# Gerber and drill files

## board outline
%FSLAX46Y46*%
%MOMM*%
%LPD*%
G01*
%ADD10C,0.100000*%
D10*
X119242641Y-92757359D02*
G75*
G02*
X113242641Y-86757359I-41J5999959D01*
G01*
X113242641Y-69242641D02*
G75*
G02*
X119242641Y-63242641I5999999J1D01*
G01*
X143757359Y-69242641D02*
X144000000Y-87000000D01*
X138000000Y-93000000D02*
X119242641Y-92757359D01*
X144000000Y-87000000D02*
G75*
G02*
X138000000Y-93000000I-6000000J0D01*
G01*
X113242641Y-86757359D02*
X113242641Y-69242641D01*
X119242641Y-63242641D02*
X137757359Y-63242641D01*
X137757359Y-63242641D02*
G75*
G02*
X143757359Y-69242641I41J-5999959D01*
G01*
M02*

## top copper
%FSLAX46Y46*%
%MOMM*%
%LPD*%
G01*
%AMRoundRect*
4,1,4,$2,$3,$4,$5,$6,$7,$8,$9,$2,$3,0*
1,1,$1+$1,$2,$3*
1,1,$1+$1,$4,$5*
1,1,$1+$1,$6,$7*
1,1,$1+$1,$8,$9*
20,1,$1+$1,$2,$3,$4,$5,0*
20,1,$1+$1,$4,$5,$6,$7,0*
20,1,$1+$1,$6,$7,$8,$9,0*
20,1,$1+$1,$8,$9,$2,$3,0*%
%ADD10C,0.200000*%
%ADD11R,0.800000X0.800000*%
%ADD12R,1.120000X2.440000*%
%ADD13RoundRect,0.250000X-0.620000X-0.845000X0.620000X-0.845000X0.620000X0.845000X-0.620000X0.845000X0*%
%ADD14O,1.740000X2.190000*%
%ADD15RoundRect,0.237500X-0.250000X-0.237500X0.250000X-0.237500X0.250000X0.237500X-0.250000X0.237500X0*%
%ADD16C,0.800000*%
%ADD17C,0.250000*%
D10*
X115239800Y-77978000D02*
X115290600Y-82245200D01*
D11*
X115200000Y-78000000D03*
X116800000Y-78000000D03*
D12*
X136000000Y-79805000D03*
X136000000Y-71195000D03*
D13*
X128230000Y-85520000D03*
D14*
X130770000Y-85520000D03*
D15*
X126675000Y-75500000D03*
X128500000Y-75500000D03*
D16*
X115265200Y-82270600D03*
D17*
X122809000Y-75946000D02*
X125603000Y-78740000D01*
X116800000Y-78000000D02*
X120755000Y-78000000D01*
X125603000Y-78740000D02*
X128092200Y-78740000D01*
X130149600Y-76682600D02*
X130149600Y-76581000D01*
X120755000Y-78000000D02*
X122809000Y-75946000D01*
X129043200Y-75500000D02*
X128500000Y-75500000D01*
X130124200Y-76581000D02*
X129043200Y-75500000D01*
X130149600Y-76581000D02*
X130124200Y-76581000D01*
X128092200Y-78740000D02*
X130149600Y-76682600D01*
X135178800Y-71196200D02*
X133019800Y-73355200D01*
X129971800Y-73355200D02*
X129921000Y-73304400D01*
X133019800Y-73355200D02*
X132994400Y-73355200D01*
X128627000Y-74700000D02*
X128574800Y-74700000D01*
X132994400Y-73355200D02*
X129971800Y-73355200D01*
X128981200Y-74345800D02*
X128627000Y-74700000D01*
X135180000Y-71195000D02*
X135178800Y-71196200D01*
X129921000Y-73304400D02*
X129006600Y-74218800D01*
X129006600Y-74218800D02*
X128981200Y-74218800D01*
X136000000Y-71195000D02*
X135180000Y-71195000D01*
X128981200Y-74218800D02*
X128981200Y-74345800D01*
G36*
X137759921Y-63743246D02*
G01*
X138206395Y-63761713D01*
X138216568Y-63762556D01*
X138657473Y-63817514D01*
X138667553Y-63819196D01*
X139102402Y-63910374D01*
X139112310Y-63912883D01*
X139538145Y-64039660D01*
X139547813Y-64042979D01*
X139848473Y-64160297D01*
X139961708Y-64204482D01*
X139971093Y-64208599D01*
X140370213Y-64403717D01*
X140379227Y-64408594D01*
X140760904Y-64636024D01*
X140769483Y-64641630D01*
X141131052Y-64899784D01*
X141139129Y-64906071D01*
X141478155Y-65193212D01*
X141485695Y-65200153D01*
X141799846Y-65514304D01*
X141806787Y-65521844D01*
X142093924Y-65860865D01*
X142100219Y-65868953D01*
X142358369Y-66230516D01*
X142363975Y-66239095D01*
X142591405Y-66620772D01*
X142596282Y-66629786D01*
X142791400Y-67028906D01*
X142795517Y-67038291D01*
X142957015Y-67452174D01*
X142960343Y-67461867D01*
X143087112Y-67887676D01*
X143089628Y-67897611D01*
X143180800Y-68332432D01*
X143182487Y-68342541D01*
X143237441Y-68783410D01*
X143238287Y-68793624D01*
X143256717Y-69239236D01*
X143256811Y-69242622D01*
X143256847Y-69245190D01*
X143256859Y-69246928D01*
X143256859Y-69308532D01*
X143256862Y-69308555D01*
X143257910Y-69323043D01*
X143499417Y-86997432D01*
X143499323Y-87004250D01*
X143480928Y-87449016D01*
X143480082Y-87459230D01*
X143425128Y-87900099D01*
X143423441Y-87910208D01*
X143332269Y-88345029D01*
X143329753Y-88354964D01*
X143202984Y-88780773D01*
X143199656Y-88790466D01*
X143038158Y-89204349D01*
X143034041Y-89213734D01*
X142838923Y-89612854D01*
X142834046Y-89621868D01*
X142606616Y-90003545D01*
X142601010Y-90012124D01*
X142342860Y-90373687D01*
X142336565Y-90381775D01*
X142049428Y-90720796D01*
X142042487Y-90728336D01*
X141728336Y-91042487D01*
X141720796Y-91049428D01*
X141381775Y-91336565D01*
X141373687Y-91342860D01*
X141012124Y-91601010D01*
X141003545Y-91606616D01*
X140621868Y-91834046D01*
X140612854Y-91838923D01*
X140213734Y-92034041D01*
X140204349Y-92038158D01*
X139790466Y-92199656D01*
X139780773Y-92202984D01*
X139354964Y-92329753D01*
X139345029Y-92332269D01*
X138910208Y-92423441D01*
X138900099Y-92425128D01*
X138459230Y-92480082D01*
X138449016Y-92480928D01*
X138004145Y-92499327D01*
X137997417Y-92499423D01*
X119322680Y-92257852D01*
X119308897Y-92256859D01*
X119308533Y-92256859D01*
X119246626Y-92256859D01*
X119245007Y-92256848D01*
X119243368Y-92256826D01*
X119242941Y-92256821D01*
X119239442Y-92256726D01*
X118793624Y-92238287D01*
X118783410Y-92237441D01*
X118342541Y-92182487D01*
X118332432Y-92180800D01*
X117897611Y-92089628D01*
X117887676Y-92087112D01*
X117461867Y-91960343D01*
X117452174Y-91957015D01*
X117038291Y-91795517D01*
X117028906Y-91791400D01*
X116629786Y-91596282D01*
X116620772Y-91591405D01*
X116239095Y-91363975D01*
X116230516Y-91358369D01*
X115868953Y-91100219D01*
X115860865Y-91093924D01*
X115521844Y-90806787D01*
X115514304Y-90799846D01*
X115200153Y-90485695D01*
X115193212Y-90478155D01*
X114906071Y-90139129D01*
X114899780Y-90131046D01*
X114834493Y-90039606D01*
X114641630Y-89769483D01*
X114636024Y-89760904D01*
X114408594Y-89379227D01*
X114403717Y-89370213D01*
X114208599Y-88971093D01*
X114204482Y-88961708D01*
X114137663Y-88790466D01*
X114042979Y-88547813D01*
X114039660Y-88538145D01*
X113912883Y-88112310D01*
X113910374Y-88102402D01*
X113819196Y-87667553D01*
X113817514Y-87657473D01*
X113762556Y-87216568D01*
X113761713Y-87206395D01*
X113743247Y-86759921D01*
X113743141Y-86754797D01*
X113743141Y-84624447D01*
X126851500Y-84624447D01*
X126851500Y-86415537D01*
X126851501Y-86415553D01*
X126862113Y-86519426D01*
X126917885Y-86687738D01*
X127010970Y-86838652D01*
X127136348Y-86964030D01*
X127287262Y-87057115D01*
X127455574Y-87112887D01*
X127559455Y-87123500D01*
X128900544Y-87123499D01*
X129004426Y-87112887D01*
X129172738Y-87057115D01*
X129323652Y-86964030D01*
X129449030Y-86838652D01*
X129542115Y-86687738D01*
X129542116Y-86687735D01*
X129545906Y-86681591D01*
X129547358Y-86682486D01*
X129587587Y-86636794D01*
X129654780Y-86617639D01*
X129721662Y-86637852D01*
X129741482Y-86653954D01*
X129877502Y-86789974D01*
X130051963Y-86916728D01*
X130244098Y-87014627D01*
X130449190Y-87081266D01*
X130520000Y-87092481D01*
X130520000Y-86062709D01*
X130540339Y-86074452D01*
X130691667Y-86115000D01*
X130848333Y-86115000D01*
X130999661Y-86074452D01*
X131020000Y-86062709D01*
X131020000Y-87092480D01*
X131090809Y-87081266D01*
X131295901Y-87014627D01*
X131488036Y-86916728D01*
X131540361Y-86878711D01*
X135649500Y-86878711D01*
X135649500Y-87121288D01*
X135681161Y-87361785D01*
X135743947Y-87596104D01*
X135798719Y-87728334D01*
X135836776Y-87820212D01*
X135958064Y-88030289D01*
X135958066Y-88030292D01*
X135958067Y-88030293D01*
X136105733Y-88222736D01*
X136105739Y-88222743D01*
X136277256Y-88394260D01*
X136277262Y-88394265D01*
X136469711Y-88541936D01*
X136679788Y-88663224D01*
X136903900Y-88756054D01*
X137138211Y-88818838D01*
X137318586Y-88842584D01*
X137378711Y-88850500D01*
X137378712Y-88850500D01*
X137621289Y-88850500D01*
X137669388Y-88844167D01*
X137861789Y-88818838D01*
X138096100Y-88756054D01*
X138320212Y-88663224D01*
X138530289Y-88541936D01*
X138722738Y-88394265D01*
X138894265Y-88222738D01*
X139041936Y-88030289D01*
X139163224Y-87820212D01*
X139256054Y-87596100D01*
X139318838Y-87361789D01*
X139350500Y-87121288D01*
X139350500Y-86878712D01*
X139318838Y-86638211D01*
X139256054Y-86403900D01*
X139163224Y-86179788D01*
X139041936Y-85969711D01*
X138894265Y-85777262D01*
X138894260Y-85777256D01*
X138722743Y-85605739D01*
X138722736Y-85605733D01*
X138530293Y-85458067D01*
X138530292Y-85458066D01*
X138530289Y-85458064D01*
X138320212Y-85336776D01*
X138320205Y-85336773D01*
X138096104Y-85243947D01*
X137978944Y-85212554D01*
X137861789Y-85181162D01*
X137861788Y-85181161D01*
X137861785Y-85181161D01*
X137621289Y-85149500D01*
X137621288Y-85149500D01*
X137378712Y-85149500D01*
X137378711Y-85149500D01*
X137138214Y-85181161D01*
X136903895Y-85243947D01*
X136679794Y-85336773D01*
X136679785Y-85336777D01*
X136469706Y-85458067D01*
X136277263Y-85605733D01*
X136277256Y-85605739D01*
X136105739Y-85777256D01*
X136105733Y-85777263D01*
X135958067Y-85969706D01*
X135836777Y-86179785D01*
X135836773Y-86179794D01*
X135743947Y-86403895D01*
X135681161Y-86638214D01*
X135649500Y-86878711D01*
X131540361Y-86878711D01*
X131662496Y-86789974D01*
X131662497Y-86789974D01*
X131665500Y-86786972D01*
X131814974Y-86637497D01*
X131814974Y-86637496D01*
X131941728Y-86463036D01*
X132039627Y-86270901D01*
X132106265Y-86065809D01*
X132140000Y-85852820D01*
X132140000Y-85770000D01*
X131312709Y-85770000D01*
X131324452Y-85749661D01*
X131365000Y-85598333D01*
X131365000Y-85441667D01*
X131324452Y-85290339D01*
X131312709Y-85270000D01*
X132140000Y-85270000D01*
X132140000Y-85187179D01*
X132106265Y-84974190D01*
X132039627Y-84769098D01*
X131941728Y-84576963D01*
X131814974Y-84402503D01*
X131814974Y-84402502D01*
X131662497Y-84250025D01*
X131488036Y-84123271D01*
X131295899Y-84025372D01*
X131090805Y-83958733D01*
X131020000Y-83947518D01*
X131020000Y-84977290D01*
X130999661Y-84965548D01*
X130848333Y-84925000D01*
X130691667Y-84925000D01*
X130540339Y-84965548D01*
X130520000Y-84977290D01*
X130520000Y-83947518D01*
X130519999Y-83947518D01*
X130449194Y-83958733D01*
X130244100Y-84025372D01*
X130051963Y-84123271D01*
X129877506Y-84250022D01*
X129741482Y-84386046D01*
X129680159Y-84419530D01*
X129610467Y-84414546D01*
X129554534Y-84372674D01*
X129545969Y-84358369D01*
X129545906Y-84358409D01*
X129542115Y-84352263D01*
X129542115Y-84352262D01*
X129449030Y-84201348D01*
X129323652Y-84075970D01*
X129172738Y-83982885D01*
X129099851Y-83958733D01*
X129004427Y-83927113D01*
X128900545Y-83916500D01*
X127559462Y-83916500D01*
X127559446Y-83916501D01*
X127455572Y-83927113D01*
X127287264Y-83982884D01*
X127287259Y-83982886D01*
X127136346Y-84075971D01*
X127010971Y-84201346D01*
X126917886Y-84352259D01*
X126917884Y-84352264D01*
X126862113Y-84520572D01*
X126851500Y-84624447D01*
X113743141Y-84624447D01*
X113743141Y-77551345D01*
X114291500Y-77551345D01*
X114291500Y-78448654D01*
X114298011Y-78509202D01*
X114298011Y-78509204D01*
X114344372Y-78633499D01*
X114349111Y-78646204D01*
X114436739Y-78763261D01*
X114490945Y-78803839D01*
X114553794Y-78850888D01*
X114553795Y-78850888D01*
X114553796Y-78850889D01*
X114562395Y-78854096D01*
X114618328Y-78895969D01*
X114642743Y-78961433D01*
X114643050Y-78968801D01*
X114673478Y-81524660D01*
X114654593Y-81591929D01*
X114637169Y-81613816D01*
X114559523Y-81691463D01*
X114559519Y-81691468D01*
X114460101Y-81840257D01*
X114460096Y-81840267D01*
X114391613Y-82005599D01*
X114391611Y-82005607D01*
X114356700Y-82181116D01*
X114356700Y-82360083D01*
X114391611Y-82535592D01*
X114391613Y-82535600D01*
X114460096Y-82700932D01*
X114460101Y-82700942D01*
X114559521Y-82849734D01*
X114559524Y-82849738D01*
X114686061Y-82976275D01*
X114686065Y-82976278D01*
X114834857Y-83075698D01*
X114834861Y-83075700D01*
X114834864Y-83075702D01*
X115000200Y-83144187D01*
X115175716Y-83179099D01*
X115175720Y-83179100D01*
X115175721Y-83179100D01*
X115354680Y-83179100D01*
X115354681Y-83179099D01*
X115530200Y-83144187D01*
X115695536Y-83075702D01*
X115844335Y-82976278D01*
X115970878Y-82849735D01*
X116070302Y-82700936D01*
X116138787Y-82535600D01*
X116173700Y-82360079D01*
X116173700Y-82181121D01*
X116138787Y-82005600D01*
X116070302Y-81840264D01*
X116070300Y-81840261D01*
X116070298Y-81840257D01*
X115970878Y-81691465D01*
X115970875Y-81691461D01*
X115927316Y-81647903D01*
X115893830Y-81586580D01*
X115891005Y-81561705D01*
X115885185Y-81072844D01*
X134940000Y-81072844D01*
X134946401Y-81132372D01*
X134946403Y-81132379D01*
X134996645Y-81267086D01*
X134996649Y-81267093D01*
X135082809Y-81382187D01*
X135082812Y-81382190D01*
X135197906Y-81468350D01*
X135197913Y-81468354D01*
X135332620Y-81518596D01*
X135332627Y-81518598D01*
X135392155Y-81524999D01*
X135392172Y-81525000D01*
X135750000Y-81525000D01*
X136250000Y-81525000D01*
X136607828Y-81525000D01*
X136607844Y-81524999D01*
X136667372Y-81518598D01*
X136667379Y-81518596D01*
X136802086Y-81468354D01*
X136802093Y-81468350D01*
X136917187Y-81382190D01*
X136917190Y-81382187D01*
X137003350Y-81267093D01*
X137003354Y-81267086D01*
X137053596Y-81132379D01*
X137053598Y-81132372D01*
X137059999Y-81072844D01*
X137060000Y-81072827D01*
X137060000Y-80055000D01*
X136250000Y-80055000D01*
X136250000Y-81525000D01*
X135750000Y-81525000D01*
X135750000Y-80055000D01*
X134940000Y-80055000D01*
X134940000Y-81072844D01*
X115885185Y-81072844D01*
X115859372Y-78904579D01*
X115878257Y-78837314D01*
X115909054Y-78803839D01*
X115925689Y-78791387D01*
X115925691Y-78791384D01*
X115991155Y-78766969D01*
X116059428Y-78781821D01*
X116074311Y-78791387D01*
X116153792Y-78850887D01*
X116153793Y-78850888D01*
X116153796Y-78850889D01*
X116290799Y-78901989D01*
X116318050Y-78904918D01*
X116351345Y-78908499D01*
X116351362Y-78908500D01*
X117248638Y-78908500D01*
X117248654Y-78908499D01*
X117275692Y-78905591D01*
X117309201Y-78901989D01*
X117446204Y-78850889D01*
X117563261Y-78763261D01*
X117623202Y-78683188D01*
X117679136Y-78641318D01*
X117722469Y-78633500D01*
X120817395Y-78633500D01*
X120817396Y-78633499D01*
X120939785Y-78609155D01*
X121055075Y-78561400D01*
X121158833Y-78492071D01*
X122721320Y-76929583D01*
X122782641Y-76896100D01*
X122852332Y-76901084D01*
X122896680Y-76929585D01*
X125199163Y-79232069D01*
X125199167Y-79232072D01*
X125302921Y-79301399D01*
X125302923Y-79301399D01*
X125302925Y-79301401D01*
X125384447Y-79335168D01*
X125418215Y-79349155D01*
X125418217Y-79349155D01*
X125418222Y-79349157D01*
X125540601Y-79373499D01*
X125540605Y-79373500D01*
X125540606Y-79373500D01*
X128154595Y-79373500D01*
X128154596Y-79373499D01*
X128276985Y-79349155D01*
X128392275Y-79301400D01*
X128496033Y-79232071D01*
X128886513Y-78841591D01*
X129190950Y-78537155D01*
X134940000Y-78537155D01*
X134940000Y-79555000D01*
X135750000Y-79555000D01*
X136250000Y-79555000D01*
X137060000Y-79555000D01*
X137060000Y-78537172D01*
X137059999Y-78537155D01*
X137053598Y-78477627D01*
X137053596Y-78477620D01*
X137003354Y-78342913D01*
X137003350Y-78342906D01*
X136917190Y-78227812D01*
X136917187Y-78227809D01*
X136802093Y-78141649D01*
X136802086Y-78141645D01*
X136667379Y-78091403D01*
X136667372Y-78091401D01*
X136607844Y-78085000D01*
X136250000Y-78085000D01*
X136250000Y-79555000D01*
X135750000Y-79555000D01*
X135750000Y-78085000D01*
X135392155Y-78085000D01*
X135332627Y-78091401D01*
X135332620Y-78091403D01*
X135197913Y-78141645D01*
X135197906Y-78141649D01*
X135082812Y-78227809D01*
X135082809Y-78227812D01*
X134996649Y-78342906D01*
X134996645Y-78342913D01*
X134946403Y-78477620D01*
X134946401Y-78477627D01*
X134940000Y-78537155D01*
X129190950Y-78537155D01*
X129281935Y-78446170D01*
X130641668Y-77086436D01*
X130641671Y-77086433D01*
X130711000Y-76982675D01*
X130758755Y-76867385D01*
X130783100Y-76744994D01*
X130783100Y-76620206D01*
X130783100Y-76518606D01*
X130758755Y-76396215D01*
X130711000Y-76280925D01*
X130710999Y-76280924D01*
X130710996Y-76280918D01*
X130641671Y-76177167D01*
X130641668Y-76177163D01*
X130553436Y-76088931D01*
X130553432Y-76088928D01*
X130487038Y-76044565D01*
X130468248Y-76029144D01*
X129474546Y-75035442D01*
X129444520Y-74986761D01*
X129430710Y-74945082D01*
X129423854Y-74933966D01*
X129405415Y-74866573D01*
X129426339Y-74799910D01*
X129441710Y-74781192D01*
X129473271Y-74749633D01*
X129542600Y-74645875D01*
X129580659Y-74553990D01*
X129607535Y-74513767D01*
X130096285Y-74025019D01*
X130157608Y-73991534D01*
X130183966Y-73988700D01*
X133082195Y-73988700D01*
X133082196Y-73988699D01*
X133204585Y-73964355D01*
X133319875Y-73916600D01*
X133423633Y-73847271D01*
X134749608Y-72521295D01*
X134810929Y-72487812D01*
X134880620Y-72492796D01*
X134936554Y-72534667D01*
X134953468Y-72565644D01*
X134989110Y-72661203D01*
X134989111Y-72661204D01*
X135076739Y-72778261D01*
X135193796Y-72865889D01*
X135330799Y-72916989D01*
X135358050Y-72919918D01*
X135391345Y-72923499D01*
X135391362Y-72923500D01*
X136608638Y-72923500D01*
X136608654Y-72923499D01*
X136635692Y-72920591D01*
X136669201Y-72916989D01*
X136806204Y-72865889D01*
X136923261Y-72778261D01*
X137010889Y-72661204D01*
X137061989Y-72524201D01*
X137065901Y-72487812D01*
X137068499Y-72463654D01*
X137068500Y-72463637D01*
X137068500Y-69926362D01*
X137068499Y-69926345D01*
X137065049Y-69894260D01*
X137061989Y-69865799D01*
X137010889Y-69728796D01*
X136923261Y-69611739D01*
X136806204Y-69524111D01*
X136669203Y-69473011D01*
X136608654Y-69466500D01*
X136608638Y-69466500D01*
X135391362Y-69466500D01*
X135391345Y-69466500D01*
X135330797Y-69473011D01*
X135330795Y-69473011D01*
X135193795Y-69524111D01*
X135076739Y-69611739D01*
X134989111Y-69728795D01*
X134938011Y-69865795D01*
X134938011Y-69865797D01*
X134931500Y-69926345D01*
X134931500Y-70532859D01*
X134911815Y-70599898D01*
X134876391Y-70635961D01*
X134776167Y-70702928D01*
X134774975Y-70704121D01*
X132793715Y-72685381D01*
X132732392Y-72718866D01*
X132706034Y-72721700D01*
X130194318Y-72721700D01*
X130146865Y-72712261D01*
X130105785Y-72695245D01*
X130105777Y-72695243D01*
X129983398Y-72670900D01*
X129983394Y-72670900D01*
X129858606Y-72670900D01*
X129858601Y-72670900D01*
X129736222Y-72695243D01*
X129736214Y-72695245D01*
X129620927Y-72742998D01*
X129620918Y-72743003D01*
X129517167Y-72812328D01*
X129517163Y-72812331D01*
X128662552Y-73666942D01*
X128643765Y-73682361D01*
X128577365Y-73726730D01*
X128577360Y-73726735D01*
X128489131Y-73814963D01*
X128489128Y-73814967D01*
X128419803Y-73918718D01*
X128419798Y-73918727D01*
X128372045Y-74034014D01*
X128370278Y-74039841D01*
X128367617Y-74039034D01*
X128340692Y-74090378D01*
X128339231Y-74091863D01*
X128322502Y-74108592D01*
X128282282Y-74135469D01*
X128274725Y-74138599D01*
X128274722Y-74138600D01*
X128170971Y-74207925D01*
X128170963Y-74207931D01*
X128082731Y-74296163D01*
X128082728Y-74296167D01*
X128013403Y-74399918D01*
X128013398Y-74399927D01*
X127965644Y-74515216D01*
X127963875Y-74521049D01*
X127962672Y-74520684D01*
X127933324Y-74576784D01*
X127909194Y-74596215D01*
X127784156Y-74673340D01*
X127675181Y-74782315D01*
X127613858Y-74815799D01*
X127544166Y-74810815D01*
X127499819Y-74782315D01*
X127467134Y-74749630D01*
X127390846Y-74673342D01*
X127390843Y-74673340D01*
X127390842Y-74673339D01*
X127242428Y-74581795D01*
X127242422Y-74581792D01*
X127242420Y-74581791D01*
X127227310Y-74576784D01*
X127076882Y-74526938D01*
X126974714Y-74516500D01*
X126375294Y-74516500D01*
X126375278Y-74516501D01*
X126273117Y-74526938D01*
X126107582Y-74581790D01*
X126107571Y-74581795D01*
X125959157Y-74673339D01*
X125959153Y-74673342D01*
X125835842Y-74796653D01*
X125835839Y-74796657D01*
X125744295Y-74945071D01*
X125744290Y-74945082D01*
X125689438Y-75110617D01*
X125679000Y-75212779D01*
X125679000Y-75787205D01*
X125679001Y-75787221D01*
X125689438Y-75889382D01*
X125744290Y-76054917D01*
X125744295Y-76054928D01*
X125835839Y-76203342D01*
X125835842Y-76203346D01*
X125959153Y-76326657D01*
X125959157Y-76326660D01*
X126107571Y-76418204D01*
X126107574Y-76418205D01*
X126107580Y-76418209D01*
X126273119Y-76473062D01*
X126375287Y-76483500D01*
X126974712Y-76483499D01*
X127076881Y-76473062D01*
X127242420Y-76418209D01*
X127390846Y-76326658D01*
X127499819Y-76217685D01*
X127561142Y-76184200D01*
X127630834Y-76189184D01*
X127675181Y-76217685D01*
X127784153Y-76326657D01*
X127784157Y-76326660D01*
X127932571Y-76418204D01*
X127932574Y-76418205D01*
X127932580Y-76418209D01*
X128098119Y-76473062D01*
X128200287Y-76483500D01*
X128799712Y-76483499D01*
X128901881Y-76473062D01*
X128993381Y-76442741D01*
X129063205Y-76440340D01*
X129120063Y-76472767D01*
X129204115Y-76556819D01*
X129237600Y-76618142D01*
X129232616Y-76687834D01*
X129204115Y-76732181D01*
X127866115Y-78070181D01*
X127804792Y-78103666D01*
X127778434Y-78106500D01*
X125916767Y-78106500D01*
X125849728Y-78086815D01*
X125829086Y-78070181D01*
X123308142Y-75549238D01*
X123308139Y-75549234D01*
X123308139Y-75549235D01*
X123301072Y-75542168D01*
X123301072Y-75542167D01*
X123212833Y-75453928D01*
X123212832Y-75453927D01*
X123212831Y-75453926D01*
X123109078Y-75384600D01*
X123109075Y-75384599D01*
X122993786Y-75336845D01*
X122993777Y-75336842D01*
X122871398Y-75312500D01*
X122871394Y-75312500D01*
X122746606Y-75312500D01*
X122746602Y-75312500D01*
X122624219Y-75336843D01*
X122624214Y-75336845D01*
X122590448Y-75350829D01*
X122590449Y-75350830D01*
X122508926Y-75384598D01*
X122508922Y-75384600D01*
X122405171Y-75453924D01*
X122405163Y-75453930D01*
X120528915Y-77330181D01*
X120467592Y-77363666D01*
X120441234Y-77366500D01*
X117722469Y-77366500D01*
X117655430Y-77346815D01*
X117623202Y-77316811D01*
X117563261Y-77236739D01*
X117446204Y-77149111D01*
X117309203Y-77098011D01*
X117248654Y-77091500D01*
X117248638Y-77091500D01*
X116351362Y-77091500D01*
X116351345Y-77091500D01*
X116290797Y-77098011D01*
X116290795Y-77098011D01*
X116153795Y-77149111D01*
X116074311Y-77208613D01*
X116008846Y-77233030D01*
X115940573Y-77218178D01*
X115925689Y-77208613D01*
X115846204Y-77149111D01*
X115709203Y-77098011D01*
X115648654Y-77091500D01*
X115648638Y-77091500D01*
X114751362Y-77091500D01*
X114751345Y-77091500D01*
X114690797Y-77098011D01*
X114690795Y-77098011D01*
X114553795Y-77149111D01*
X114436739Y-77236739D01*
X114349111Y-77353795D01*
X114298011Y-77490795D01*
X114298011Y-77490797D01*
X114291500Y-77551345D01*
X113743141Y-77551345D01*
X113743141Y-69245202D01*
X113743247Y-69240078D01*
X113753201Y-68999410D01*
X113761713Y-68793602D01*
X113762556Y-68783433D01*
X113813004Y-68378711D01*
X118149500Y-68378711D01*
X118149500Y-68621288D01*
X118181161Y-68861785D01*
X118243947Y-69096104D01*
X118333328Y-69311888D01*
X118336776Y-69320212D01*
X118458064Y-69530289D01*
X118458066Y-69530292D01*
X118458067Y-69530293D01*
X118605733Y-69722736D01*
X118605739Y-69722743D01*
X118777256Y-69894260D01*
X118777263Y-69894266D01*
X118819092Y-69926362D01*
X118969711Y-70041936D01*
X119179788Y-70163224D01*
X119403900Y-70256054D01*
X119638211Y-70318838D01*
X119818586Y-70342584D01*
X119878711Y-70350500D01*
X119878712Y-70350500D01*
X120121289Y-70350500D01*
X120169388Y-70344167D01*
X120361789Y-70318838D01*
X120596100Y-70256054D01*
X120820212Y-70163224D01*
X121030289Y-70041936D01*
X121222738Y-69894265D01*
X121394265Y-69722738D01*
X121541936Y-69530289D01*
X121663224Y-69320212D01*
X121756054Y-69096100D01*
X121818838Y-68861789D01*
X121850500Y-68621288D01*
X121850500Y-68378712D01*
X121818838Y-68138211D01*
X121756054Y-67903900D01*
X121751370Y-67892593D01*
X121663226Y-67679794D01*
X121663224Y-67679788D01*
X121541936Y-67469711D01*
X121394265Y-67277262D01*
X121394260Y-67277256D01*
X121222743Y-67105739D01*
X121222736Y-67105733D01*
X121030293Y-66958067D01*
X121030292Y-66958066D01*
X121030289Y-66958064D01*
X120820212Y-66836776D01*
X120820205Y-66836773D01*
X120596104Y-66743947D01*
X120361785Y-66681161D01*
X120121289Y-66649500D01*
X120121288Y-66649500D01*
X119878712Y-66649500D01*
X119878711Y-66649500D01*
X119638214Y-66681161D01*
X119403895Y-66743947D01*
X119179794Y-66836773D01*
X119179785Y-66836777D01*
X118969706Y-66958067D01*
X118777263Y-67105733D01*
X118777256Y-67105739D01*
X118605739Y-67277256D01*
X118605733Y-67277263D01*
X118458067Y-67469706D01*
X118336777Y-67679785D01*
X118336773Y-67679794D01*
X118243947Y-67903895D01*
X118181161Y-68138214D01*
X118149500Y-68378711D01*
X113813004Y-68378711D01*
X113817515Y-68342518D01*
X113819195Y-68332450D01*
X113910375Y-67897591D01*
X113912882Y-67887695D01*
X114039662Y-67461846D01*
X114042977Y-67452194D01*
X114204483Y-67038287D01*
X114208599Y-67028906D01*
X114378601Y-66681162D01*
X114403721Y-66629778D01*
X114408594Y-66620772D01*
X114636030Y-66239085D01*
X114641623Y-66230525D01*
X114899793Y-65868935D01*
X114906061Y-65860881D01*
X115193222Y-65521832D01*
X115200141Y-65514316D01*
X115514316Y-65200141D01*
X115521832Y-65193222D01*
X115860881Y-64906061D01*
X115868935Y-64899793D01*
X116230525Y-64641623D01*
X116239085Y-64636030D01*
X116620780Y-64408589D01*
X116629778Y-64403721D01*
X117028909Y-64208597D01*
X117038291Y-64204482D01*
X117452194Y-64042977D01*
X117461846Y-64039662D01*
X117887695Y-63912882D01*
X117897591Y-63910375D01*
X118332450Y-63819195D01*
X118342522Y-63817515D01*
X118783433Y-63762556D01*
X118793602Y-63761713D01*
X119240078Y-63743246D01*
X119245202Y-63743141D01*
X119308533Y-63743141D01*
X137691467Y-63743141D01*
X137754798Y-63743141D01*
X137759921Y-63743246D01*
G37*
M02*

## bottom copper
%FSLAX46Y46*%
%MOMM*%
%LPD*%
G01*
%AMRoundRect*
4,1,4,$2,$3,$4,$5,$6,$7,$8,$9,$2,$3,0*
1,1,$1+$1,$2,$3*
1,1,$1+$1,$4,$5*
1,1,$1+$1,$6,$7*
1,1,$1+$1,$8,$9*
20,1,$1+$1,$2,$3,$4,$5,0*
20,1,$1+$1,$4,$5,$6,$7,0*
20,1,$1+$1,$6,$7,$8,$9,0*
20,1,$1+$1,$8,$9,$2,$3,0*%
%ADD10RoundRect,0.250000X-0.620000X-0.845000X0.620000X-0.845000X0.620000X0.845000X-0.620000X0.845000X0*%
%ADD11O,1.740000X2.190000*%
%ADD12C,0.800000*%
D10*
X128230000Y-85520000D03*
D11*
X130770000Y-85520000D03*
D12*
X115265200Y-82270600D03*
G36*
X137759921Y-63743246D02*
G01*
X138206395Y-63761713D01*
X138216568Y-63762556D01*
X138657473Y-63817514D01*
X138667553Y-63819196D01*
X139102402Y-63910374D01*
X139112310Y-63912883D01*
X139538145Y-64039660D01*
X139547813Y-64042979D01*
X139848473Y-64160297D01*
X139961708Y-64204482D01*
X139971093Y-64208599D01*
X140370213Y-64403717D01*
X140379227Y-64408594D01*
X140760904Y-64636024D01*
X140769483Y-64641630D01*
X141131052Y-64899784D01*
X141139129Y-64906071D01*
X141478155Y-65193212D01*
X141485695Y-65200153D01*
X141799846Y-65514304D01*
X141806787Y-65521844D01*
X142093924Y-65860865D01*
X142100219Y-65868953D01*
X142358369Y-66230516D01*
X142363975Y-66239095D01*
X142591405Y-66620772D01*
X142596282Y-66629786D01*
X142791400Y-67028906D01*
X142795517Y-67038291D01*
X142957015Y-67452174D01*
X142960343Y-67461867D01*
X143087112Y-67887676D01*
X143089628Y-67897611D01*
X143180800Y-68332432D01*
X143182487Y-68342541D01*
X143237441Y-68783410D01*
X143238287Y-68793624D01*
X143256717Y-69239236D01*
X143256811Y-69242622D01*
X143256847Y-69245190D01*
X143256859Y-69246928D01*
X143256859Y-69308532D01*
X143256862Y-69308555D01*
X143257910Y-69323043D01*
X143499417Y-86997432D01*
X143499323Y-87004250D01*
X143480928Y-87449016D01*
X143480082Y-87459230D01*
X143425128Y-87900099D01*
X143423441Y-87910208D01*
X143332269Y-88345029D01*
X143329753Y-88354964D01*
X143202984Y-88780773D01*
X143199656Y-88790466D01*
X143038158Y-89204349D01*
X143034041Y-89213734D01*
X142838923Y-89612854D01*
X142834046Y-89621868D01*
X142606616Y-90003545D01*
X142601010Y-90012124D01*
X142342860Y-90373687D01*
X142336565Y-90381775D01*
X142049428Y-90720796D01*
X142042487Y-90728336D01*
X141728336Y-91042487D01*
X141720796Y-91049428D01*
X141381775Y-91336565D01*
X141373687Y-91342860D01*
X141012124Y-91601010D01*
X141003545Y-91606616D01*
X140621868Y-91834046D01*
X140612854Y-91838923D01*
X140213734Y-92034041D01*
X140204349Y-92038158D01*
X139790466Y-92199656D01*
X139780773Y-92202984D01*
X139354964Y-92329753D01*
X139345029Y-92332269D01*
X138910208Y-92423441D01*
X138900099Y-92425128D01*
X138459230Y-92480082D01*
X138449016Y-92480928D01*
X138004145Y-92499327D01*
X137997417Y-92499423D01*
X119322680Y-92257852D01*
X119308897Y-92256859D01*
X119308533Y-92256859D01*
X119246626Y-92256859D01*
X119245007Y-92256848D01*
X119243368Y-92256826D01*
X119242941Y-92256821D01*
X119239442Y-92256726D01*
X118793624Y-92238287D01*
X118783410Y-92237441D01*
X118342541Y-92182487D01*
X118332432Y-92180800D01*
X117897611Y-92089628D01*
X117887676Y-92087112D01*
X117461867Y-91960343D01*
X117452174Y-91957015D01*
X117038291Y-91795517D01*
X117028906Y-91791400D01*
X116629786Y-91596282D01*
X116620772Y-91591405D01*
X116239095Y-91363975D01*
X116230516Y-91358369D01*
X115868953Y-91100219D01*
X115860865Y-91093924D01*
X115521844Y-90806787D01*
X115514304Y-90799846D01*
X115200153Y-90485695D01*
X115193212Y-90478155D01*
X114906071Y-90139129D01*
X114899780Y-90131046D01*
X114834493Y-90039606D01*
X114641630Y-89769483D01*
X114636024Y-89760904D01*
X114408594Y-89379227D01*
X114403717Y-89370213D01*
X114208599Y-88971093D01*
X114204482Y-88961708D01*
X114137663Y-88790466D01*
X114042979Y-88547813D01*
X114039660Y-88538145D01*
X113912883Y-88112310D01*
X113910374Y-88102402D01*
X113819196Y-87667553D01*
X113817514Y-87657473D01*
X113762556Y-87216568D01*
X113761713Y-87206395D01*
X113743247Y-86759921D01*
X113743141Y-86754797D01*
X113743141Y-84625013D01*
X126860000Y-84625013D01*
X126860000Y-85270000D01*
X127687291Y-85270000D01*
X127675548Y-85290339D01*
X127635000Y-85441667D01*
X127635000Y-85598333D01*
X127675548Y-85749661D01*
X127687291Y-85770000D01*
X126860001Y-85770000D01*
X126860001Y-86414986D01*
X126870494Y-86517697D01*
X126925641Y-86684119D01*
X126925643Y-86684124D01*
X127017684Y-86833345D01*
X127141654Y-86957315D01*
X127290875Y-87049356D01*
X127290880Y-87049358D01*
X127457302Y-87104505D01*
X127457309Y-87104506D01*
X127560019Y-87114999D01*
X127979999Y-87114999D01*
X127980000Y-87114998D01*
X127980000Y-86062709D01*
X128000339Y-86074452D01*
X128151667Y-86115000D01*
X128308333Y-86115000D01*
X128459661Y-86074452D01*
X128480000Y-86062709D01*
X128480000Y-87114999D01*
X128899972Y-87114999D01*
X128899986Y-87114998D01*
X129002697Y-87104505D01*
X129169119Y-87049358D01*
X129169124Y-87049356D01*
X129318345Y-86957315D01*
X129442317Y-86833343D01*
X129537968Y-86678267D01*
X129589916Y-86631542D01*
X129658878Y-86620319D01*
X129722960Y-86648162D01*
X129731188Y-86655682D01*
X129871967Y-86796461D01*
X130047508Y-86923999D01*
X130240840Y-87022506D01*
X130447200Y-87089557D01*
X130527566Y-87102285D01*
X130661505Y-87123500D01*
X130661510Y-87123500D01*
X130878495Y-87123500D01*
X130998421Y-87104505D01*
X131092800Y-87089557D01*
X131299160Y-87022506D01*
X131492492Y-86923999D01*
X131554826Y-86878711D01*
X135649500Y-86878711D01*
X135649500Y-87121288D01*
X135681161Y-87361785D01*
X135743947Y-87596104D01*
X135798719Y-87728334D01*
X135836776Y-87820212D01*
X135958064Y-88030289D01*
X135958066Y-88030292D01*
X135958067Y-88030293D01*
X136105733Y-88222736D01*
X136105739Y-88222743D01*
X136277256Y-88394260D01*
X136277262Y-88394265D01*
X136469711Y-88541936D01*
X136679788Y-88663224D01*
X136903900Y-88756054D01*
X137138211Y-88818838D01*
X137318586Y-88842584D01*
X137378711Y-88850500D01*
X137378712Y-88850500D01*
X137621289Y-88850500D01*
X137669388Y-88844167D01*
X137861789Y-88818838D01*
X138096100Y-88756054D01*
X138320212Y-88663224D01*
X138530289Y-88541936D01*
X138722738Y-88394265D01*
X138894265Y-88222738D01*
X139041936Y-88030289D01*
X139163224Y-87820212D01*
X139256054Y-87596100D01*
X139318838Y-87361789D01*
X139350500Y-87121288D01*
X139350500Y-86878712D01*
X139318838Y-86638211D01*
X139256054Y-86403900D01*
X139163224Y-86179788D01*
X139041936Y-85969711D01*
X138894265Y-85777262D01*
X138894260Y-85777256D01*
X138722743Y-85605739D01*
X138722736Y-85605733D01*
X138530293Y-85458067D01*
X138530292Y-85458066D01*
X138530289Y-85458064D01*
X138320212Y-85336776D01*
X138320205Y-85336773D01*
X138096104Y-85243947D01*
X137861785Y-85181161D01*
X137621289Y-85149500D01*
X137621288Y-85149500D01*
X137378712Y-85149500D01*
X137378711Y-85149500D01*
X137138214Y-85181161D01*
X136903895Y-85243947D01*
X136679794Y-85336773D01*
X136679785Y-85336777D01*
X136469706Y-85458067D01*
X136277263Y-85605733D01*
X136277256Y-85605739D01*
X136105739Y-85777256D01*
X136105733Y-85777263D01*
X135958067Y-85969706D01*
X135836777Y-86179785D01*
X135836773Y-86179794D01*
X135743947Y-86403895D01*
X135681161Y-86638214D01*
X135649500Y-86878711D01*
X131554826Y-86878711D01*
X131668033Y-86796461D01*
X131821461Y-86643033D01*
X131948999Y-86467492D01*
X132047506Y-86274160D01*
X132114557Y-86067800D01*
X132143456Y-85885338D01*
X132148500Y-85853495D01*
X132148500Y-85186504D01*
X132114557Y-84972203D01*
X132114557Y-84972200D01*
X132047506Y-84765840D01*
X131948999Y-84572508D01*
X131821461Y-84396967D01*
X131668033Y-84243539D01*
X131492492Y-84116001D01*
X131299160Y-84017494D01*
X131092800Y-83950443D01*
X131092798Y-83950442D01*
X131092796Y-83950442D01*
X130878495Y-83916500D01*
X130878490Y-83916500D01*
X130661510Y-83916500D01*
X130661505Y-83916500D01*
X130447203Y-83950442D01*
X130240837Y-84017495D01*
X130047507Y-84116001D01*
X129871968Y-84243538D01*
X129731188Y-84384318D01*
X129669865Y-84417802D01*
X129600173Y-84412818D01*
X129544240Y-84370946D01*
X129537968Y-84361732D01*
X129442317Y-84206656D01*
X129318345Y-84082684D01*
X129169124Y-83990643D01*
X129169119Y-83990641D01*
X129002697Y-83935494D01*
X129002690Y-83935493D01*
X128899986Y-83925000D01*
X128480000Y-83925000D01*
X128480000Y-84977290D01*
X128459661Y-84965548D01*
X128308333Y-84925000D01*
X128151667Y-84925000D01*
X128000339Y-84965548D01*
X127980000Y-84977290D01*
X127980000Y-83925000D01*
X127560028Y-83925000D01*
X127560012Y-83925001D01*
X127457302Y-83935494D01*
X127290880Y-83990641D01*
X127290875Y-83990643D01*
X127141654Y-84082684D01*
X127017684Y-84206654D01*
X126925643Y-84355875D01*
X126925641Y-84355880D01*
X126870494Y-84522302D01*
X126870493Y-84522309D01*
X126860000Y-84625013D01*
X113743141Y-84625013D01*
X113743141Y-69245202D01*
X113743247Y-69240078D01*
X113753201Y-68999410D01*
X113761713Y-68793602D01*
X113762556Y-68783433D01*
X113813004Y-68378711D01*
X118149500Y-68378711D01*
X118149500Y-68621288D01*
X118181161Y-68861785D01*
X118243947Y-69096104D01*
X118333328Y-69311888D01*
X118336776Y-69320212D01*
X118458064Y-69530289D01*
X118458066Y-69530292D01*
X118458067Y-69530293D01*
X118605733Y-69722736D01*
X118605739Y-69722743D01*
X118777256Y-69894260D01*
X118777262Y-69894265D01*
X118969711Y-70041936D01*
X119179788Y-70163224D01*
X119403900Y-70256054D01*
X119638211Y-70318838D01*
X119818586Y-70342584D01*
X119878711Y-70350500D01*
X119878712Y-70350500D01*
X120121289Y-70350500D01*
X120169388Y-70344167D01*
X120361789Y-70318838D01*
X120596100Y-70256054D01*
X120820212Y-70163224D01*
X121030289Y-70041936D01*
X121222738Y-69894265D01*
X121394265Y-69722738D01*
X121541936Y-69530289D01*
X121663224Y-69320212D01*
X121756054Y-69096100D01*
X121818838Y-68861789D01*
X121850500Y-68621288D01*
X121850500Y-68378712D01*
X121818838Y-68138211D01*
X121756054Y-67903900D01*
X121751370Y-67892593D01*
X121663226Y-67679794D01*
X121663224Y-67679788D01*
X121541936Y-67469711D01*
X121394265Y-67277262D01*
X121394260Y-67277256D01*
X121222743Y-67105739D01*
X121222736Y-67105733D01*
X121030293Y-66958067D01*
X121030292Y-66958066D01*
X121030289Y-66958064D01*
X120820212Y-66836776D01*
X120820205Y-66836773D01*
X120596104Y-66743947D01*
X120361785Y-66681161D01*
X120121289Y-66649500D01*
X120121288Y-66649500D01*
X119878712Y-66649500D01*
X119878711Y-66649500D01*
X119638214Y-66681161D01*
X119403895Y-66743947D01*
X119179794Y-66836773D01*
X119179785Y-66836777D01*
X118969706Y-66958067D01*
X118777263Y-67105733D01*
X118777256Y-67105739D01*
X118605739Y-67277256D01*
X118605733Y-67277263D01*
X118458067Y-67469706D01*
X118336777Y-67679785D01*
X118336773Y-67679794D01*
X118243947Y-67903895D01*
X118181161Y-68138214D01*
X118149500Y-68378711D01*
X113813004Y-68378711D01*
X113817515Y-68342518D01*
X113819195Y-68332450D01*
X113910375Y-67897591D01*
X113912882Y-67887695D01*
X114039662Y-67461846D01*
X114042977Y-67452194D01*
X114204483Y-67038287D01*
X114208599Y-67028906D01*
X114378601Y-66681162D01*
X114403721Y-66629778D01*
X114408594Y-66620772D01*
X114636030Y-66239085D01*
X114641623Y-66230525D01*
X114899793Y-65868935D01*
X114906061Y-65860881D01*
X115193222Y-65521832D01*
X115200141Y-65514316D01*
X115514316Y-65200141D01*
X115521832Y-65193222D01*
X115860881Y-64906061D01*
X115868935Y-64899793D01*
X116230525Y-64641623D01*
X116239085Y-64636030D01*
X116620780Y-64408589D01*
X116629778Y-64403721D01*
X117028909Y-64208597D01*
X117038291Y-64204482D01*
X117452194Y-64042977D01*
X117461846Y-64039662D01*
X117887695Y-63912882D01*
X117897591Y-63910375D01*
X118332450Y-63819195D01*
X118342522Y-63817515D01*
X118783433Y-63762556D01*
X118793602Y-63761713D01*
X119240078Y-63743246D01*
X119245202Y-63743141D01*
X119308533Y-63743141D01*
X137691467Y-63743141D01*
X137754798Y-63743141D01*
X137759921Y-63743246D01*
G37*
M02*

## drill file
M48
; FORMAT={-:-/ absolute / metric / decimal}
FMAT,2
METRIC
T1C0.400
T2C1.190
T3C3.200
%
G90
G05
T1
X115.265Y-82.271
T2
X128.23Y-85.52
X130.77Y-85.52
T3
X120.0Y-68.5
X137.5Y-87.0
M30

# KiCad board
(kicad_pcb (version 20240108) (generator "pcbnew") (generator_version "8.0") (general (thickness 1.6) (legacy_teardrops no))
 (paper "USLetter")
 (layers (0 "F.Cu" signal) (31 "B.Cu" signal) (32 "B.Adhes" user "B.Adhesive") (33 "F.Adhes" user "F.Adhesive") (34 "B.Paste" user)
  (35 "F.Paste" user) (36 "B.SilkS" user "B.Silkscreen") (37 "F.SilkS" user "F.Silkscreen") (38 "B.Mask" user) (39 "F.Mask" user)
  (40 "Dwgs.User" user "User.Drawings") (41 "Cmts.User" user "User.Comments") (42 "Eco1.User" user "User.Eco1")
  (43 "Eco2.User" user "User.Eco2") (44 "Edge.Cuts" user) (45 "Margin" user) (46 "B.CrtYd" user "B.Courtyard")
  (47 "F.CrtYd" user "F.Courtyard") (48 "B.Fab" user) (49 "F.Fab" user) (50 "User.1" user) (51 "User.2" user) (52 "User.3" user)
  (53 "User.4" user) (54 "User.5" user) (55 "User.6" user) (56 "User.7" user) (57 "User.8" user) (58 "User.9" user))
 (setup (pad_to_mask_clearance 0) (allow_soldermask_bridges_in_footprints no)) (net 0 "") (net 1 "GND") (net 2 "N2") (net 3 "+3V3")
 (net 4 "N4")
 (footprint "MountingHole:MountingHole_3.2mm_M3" (layer "F.Cu") (at 120 68.5)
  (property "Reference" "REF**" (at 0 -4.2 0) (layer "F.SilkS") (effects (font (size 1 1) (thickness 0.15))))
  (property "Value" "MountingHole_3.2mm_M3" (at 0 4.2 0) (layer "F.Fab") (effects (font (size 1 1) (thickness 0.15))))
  (pad "" np_thru_hole circle (at 0 0) (size 3.2 3.2) (drill 3.2) (layers "*.Cu" "*.Mask")))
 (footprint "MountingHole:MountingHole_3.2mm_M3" (layer "F.Cu") (at 137.5 87)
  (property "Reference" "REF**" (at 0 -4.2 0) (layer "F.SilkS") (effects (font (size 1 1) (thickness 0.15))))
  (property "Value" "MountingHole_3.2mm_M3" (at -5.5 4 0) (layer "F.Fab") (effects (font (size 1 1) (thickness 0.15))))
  (pad "" np_thru_hole circle (at 0 0) (size 3.2 3.2) (drill 3.2) (layers "*.Cu" "*.Mask")))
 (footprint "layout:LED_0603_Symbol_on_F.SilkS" (layer "F.Cu") (at 116 78)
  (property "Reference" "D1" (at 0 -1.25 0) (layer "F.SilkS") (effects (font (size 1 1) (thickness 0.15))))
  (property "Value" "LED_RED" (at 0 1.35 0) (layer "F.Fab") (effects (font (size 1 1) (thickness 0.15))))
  (pad "1" smd rect (at -0.8 0 180) (size 0.8 0.8) (layers "F.Cu" "F.Paste" "F.Mask") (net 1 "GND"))
  (pad "2" smd rect (at 0.8 0 180) (size 0.8 0.8) (layers "F.Cu" "F.Paste" "F.Mask") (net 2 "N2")))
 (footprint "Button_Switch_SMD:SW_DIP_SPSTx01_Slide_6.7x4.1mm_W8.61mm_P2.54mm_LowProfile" (layer "F.Cu") (at 136 75.5 90)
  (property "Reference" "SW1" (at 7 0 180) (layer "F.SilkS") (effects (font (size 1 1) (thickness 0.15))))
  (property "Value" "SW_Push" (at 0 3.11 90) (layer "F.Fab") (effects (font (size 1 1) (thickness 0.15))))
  (pad "1" smd rect (at -4.305 0 90) (size 2.44 1.12) (layers "F.Cu" "F.Paste" "F.Mask") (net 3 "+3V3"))
  (pad "2" smd rect (at 4.305 0 90) (size 2.44 1.12) (layers "F.Cu" "F.Paste" "F.Mask") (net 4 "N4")))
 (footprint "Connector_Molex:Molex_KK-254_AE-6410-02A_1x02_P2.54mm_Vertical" (layer "F.Cu") (at 128.23 85.52)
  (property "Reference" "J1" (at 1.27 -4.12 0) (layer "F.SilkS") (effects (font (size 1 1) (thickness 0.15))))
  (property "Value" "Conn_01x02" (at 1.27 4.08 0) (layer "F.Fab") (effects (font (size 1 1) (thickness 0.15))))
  (pad "1" thru_hole roundrect (at 0 0) (size 1.74 2.19) (drill 1.19) (layers "*.Cu" "*.Mask") (remove_unused_layers no)
   (roundrect_rratio 0.143678) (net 1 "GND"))
  (pad "2" thru_hole oval (at 2.54 0) (size 1.74 2.19) (drill 1.19) (layers "*.Cu" "*.Mask") (remove_unused_layers no) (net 3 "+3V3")))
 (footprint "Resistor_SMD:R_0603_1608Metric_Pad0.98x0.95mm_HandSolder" (layer "F.Cu") (at 127.5875 75.5)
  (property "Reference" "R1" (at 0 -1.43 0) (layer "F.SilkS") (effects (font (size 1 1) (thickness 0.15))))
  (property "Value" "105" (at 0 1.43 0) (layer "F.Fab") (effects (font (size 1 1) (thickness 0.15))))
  (pad "1" smd roundrect (at -0.9125 0) (size 0.975 0.95) (layers "F.Cu" "F.Paste" "F.Mask") (roundrect_rratio 0.25) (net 4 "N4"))
  (pad "2" smd roundrect (at 0.9125 0) (size 0.975 0.95) (layers "F.Cu" "F.Paste" "F.Mask") (roundrect_rratio 0.25) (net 2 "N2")))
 (gr_line (start 115.2398 77.978) (end 115.2906 82.2452) (stroke (width 0.2) (type default)) (layer "F.Cu") (net 1))
 (gr_arc (start 119.242641 92.757359) (mid 115 91) (end 113.242641 86.757359) (stroke (width 0.1) (type default)) (layer "Edge.Cuts"))
 (gr_arc (start 113.242641 69.242641) (mid 115 65) (end 119.242641 63.242641) (stroke (width 0.1) (type default)) (layer "Edge.Cuts"))
 (gr_line (start 143.757359 69.242641) (end 144 87) (stroke (width 0.1) (type default)) (layer "Edge.Cuts"))
 (gr_line (start 138 93) (end 119.242641 92.757359) (stroke (width 0.1) (type default)) (layer "Edge.Cuts"))
 (gr_arc (start 144 87) (mid 142.242641 91.242641) (end 138 93) (stroke (width 0.1) (type default)) (layer "Edge.Cuts"))
 (gr_line (start 113.242641 86.757359) (end 113.242641 69.242641) (stroke (width 0.1) (type default)) (layer "Edge.Cuts"))
 (gr_line (start 119.242641 63.242641) (end 137.757359 63.242641) (stroke (width 0.1) (type default)) (layer "Edge.Cuts"))
 (gr_arc (start 137.757359 63.242641) (mid 142 65) (end 143.757359 69.242641) (stroke (width 0.1) (type default)) (layer "Edge.Cuts"))
 (via (at 115.2652 82.2706) (size 0.8) (drill 0.4) (layers "F.Cu" "B.Cu") (free yes) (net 1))
 (segment (start 122.809 75.946) (end 125.603 78.74) (width 0.25) (layer "F.Cu") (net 2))
 (segment (start 116.8 78) (end 120.755 78) (width 0.25) (layer "F.Cu") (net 2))
 (segment (start 125.603 78.74) (end 128.0922 78.74) (width 0.25) (layer "F.Cu") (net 2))
 (segment (start 130.1496 76.6826) (end 130.1496 76.581) (width 0.25) (layer "F.Cu") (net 2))
 (segment (start 120.755 78) (end 122.809 75.946) (width 0.25) (layer "F.Cu") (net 2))
 (segment (start 129.0432 75.5) (end 128.5 75.5) (width 0.25) (layer "F.Cu") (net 2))
 (segment (start 130.1242 76.581) (end 129.0432 75.5) (width 0.25) (layer "F.Cu") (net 2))
 (segment (start 130.1496 76.581) (end 130.1242 76.581) (width 0.25) (layer "F.Cu") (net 2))
 (segment (start 128.0922 78.74) (end 130.1496 76.6826) (width 0.25) (layer "F.Cu") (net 2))
 (segment (start 135.1788 71.1962) (end 133.0198 73.3552) (width 0.25) (layer "F.Cu") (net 4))
 (segment (start 129.9718 73.3552) (end 129.921 73.3044) (width 0.25) (layer "F.Cu") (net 4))
 (segment (start 133.0198 73.3552) (end 132.9944 73.3552) (width 0.25) (layer "F.Cu") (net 4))
 (segment (start 128.627 74.7) (end 128.5748 74.7) (width 0.25) (layer "F.Cu") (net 4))
 (segment (start 132.9944 73.3552) (end 129.9718 73.3552) (width 0.25) (layer "F.Cu") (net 4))
 (segment (start 128.9812 74.3458) (end 128.627 74.7) (width 0.25) (layer "F.Cu") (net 4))
 (segment (start 135.18 71.195) (end 135.1788 71.1962) (width 0.25) (layer "F.Cu") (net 4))
 (segment (start 129.921 73.3044) (end 129.0066 74.2188) (width 0.25) (layer "F.Cu") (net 4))
 (segment (start 129.0066 74.2188) (end 128.9812 74.2188) (width 0.25) (layer "F.Cu") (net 4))
 (segment (start 136 71.195) (end 135.18 71.195) (width 0.25) (layer "F.Cu") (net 4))
 (segment (start 128.9812 74.2188) (end 128.9812 74.3458) (width 0.25) (layer "F.Cu") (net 4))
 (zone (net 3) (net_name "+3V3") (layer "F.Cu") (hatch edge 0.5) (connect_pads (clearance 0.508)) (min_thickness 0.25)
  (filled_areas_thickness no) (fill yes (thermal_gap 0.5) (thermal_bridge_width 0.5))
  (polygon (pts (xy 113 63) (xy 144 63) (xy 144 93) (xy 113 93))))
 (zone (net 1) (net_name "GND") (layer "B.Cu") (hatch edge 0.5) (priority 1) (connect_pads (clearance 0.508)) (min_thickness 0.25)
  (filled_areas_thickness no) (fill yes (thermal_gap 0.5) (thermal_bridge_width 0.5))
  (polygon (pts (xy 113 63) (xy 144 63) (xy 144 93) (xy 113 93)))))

